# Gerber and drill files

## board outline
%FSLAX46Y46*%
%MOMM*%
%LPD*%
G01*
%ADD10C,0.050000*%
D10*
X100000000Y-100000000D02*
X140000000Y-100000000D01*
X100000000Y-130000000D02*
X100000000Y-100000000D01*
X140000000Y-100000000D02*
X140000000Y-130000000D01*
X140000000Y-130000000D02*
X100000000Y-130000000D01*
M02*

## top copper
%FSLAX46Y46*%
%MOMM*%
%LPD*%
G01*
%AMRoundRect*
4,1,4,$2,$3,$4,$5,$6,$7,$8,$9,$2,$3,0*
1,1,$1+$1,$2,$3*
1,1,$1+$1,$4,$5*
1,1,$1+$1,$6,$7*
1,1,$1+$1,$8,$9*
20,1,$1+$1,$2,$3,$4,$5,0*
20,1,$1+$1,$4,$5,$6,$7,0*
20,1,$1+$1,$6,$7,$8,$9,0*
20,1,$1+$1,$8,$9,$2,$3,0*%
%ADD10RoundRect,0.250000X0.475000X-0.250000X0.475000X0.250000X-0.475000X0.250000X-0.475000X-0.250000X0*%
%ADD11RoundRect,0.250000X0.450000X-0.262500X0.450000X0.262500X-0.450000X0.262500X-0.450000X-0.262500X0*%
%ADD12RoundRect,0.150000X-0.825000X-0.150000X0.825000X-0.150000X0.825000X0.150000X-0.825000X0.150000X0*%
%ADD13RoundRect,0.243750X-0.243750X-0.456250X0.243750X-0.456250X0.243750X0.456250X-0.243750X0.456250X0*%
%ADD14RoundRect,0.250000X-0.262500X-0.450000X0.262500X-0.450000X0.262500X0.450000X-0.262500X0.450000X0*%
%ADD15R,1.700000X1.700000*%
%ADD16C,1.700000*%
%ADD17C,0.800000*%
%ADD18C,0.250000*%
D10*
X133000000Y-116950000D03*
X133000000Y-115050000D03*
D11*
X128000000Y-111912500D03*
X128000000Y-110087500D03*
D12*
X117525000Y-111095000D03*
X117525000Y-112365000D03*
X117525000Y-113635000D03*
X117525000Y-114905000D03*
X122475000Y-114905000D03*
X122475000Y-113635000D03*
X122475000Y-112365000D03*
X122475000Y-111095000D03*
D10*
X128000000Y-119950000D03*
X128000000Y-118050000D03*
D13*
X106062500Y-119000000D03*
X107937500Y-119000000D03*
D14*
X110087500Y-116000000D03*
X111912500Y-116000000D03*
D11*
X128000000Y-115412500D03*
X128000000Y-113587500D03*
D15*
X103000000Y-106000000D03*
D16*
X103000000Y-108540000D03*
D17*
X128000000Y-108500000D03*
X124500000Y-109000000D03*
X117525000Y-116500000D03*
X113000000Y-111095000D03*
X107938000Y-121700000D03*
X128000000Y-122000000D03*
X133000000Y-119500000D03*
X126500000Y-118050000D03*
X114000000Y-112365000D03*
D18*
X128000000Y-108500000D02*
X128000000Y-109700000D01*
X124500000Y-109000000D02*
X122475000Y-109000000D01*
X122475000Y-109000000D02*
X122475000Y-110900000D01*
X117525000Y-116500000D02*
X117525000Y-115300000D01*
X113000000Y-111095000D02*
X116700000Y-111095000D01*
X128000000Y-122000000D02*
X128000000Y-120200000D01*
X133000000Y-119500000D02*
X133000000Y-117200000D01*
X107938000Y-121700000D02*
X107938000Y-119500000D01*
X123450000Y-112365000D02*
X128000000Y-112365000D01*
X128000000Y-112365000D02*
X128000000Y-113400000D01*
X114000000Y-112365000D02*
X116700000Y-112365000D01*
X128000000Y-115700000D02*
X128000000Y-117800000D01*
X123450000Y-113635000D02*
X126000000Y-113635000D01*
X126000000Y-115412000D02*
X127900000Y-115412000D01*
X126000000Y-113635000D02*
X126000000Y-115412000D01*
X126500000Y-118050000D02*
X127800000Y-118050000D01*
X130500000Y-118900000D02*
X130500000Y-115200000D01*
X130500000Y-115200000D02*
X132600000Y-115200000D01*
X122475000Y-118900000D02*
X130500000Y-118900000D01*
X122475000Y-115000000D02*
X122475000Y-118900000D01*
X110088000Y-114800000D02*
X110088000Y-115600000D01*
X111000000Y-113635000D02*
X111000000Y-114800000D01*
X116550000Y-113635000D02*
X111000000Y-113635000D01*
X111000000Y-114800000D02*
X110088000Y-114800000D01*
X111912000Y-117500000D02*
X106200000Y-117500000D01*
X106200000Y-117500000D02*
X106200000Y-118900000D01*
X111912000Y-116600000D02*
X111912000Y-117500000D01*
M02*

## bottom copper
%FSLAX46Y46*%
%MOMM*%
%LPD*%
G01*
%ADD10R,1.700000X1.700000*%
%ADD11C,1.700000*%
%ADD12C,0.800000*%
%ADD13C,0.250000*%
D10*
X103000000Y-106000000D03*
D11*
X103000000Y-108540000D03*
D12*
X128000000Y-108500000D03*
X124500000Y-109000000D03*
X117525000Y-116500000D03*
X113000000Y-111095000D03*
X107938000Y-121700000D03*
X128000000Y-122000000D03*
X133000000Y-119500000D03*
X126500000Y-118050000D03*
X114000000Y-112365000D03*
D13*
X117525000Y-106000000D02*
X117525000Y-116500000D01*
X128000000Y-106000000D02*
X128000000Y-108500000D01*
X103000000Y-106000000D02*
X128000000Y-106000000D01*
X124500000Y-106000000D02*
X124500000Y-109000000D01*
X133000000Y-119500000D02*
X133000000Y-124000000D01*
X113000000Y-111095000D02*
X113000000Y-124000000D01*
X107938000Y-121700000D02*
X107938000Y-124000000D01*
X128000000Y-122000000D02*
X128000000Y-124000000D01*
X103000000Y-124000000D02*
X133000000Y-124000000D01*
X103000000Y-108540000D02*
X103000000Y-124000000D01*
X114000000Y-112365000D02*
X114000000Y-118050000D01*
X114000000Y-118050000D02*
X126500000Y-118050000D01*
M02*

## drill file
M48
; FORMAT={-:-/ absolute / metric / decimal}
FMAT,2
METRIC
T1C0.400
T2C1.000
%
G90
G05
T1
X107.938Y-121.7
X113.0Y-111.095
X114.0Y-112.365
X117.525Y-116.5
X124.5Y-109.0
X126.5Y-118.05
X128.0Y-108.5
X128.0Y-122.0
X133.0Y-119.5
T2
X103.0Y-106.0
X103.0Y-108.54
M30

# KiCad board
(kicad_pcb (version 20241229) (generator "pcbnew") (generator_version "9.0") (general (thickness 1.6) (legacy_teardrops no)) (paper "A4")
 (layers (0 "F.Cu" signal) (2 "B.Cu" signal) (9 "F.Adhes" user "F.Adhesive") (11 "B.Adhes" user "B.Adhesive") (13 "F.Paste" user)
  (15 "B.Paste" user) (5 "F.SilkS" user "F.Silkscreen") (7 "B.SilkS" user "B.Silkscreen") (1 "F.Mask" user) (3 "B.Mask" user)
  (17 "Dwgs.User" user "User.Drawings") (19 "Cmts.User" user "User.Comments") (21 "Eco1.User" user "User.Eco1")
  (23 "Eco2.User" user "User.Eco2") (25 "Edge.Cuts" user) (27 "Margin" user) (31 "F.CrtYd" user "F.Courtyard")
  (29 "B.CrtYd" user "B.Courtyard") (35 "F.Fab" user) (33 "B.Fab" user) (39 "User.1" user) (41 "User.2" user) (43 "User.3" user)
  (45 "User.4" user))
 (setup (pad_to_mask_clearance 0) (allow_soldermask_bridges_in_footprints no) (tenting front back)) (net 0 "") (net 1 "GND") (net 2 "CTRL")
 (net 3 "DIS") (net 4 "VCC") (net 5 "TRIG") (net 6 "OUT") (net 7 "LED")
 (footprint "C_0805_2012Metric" (layer "F.Cu") (at 133 116 90)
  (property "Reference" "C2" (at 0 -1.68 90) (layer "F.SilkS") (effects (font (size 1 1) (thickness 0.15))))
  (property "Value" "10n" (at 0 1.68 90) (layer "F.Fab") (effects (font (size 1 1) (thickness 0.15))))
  (pad "1" smd roundrect (at -0.95 0 90) (size 1 1.45) (layers "F.Cu" "F.Mask" "F.Paste") (roundrect_rratio 0.25) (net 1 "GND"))
  (pad "2" smd roundrect (at 0.95 0 90) (size 1 1.45) (layers "F.Cu" "F.Mask" "F.Paste") (roundrect_rratio 0.25) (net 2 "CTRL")))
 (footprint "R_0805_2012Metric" (layer "F.Cu") (at 128 111 90)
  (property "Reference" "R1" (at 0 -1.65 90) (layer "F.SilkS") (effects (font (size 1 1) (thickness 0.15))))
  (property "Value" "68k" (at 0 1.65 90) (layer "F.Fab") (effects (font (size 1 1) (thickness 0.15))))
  (pad "1" smd roundrect (at -0.9125 0 90) (size 1.025 1.4) (layers "F.Cu" "F.Mask" "F.Paste") (roundrect_rratio 0.243902) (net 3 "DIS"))
  (pad "2" smd roundrect (at 0.9125 0 90) (size 1.025 1.4) (layers "F.Cu" "F.Mask" "F.Paste") (roundrect_rratio 0.243902) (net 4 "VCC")))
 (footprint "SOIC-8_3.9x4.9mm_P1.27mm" (layer "F.Cu") (at 120 113)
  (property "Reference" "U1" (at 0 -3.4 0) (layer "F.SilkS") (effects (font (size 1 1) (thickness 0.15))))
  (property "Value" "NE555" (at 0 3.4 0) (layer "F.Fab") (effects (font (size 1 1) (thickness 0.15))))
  (pad "1" smd roundrect (at -2.475 -1.905) (size 1.95 0.6) (layers "F.Cu" "F.Mask" "F.Paste") (roundrect_rratio 0.25) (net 1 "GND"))
  (pad "2" smd roundrect (at -2.475 -0.635) (size 1.95 0.6) (layers "F.Cu" "F.Mask" "F.Paste") (roundrect_rratio 0.25) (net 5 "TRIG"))
  (pad "3" smd roundrect (at -2.475 0.635) (size 1.95 0.6) (layers "F.Cu" "F.Mask" "F.Paste") (roundrect_rratio 0.25) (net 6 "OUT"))
  (pad "4" smd roundrect (at -2.475 1.905) (size 1.95 0.6) (layers "F.Cu" "F.Mask" "F.Paste") (roundrect_rratio 0.25) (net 4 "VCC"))
  (pad "5" smd roundrect (at 2.475 1.905) (size 1.95 0.6) (layers "F.Cu" "F.Mask" "F.Paste") (roundrect_rratio 0.25) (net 2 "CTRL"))
  (pad "6" smd roundrect (at 2.475 0.635) (size 1.95 0.6) (layers "F.Cu" "F.Mask" "F.Paste") (roundrect_rratio 0.25) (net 5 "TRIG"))
  (pad "7" smd roundrect (at 2.475 -0.635) (size 1.95 0.6) (layers "F.Cu" "F.Mask" "F.Paste") (roundrect_rratio 0.25) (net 3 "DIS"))
  (pad "8" smd roundrect (at 2.475 -1.905) (size 1.95 0.6) (layers "F.Cu" "F.Mask" "F.Paste") (roundrect_rratio 0.25) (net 4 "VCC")))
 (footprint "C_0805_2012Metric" (layer "F.Cu") (at 128 119 90)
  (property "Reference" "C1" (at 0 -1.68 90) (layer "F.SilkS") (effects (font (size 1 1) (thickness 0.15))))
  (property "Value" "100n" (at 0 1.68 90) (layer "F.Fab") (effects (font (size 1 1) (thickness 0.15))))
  (pad "1" smd roundrect (at -0.95 0 90) (size 1 1.45) (layers "F.Cu" "F.Mask" "F.Paste") (roundrect_rratio 0.25) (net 1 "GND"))
  (pad "2" smd roundrect (at 0.95 0 90) (size 1 1.45) (layers "F.Cu" "F.Mask" "F.Paste") (roundrect_rratio 0.25) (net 5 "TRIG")))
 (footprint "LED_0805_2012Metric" (layer "F.Cu") (at 107 119)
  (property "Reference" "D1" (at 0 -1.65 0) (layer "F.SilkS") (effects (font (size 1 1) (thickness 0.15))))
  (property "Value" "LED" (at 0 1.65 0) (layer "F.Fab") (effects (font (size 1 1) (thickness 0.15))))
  (pad "1" smd roundrect (at -0.9375 0) (size 0.975 1.4) (layers "F.Cu" "F.Mask" "F.Paste") (roundrect_rratio 0.25) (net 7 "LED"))
  (pad "2" smd roundrect (at 0.9375 0) (size 0.975 1.4) (layers "F.Cu" "F.Mask" "F.Paste") (roundrect_rratio 0.25) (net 1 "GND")))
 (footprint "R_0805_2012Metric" (layer "F.Cu") (at 111 116)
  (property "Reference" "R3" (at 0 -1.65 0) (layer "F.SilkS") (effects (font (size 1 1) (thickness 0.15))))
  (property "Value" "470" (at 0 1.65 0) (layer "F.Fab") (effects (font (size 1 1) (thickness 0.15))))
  (pad "1" smd roundrect (at -0.9125 0) (size 1.025 1.4) (layers "F.Cu" "F.Mask" "F.Paste") (roundrect_rratio 0.243902) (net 6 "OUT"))
  (pad "2" smd roundrect (at 0.9125 0) (size 1.025 1.4) (layers "F.Cu" "F.Mask" "F.Paste") (roundrect_rratio 0.243902) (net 7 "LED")))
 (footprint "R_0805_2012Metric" (layer "F.Cu") (at 128 114.5 90)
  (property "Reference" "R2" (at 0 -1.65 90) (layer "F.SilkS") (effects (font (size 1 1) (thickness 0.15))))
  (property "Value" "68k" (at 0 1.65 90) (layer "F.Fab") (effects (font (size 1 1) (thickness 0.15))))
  (pad "1" smd roundrect (at -0.9125 0 90) (size 1.025 1.4) (layers "F.Cu" "F.Mask" "F.Paste") (roundrect_rratio 0.243902) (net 5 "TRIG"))
  (pad "2" smd roundrect (at 0.9125 0 90) (size 1.025 1.4) (layers "F.Cu" "F.Mask" "F.Paste") (roundrect_rratio 0.243902) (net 3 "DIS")))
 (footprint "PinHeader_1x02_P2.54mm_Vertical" (layer "F.Cu") (at 103 106)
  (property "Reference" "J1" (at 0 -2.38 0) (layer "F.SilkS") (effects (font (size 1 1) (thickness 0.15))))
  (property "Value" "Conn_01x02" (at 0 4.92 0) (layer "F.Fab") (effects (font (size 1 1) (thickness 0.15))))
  (pad "1" thru_hole rect (at 0 0) (size 1.7 1.7) (drill 1) (layers "*.Cu" "*.Mask") (remove_unused_layers no) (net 4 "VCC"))
  (pad "2" thru_hole circle (at 0 2.54) (size 1.7 1.7) (drill 1) (layers "*.Cu" "*.Mask") (remove_unused_layers no) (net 1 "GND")))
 (gr_line (start 100 100) (end 140 100) (stroke (width 0.05) (type default)) (layer "Edge.Cuts"))
 (gr_line (start 100 130) (end 100 100) (stroke (width 0.05) (type default)) (layer "Edge.Cuts"))
 (gr_line (start 140 100) (end 140 130) (stroke (width 0.05) (type default)) (layer "Edge.Cuts"))
 (gr_line (start 140 130) (end 100 130) (stroke (width 0.05) (type default)) (layer "Edge.Cuts"))
 (segment (start 128 108.5) (end 128 109.7) (width 0.25) (layer "F.Cu") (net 4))
 (segment (start 124.5 109) (end 122.475 109) (width 0.25) (layer "F.Cu") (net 4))
 (segment (start 122.475 109) (end 122.475 110.9) (width 0.25) (layer "F.Cu") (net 4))
 (segment (start 117.525 116.5) (end 117.525 115.3) (width 0.25) (layer "F.Cu") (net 4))
 (via (at 128 108.5) (size 0.8) (drill 0.4) (layers "F.Cu" "B.Cu") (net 4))
 (via (at 124.5 109) (size 0.8) (drill 0.4) (layers "F.Cu" "B.Cu") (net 4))
 (via (at 117.525 116.5) (size 0.8) (drill 0.4) (layers "F.Cu" "B.Cu") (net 4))
 (segment (start 117.525 106) (end 117.525 116.5) (width 0.25) (layer "B.Cu") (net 4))
 (segment (start 128 106) (end 128 108.5) (width 0.25) (layer "B.Cu") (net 4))
 (segment (start 103 106) (end 128 106) (width 0.25) (layer "B.Cu") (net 4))
 (segment (start 124.5 106) (end 124.5 109) (width 0.25) (layer "B.Cu") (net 4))
 (segment (start 113 111.095) (end 116.7 111.095) (width 0.25) (layer "F.Cu") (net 1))
 (segment (start 128 122) (end 128 120.2) (width 0.25) (layer "F.Cu") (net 1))
 (segment (start 133 119.5) (end 133 117.2) (width 0.25) (layer "F.Cu") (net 1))
 (segment (start 107.938 121.7) (end 107.938 119.5) (width 0.25) (layer "F.Cu") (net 1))
 (via (at 113 111.095) (size 0.8) (drill 0.4) (layers "F.Cu" "B.Cu") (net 1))
 (via (at 107.938 121.7) (size 0.8) (drill 0.4) (layers "F.Cu" "B.Cu") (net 1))
 (via (at 128 122) (size 0.8) (drill 0.4) (layers "F.Cu" "B.Cu") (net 1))
 (via (at 133 119.5) (size 0.8) (drill 0.4) (layers "F.Cu" "B.Cu") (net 1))
 (segment (start 133 119.5) (end 133 124) (width 0.25) (layer "B.Cu") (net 1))
 (segment (start 113 111.095) (end 113 124) (width 0.25) (layer "B.Cu") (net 1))
 (segment (start 107.938 121.7) (end 107.938 124) (width 0.25) (layer "B.Cu") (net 1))
 (segment (start 128 122) (end 128 124) (width 0.25) (layer "B.Cu") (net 1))
 (segment (start 103 124) (end 133 124) (width 0.25) (layer "B.Cu") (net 1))
 (segment (start 103 108.54) (end 103 124) (width 0.25) (layer "B.Cu") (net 1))
 (segment (start 123.45 112.365) (end 128 112.365) (width 0.25) (layer "F.Cu") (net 3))
 (segment (start 128 112.365) (end 128 113.4) (width 0.25) (layer "F.Cu") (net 3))
 (segment (start 114 112.365) (end 116.7 112.365) (width 0.25) (layer "F.Cu") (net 5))
 (segment (start 128 115.7) (end 128 117.8) (width 0.25) (layer "F.Cu") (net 5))
 (segment (start 123.45 113.635) (end 126 113.635) (width 0.25) (layer "F.Cu") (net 5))
 (segment (start 126 115.412) (end 127.9 115.412) (width 0.25) (layer "F.Cu") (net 5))
 (segment (start 126 113.635) (end 126 115.412) (width 0.25) (layer "F.Cu") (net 5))
 (segment (start 126.5 118.05) (end 127.8 118.05) (width 0.25) (layer "F.Cu") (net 5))
 (via (at 126.5 118.05) (size 0.8) (drill 0.4) (layers "F.Cu" "B.Cu") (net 5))
 (via (at 114 112.365) (size 0.8) (drill 0.4) (layers "F.Cu" "B.Cu") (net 5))
 (segment (start 114 112.365) (end 114 118.05) (width 0.25) (layer "B.Cu") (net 5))
 (segment (start 114 118.05) (end 126.5 118.05) (width 0.25) (layer "B.Cu") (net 5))
 (segment (start 130.5 118.9) (end 130.5 115.2) (width 0.25) (layer "F.Cu") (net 2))
 (segment (start 130.5 115.2) (end 132.6 115.2) (width 0.25) (layer "F.Cu") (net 2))
 (segment (start 122.475 118.9) (end 130.5 118.9) (width 0.25) (layer "F.Cu") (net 2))
 (segment (start 122.475 115) (end 122.475 118.9) (width 0.25) (layer "F.Cu") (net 2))
 (segment (start 110.088 114.8) (end 110.088 115.6) (width 0.25) (layer "F.Cu") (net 6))
 (segment (start 111 113.635) (end 111 114.8) (width 0.25) (layer "F.Cu") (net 6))
 (segment (start 116.55 113.635) (end 111 113.635) (width 0.25) (layer "F.Cu") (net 6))
 (segment (start 111 114.8) (end 110.088 114.8) (width 0.25) (layer "F.Cu") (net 6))
 (segment (start 111.912 117.5) (end 106.2 117.5) (width 0.25) (layer "F.Cu") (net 7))
 (segment (start 106.2 117.5) (end 106.2 118.9) (width 0.25) (layer "F.Cu") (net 7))
 (segment (start 111.912 116.6) (end 111.912 117.5) (width 0.25) (layer "F.Cu") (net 7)))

